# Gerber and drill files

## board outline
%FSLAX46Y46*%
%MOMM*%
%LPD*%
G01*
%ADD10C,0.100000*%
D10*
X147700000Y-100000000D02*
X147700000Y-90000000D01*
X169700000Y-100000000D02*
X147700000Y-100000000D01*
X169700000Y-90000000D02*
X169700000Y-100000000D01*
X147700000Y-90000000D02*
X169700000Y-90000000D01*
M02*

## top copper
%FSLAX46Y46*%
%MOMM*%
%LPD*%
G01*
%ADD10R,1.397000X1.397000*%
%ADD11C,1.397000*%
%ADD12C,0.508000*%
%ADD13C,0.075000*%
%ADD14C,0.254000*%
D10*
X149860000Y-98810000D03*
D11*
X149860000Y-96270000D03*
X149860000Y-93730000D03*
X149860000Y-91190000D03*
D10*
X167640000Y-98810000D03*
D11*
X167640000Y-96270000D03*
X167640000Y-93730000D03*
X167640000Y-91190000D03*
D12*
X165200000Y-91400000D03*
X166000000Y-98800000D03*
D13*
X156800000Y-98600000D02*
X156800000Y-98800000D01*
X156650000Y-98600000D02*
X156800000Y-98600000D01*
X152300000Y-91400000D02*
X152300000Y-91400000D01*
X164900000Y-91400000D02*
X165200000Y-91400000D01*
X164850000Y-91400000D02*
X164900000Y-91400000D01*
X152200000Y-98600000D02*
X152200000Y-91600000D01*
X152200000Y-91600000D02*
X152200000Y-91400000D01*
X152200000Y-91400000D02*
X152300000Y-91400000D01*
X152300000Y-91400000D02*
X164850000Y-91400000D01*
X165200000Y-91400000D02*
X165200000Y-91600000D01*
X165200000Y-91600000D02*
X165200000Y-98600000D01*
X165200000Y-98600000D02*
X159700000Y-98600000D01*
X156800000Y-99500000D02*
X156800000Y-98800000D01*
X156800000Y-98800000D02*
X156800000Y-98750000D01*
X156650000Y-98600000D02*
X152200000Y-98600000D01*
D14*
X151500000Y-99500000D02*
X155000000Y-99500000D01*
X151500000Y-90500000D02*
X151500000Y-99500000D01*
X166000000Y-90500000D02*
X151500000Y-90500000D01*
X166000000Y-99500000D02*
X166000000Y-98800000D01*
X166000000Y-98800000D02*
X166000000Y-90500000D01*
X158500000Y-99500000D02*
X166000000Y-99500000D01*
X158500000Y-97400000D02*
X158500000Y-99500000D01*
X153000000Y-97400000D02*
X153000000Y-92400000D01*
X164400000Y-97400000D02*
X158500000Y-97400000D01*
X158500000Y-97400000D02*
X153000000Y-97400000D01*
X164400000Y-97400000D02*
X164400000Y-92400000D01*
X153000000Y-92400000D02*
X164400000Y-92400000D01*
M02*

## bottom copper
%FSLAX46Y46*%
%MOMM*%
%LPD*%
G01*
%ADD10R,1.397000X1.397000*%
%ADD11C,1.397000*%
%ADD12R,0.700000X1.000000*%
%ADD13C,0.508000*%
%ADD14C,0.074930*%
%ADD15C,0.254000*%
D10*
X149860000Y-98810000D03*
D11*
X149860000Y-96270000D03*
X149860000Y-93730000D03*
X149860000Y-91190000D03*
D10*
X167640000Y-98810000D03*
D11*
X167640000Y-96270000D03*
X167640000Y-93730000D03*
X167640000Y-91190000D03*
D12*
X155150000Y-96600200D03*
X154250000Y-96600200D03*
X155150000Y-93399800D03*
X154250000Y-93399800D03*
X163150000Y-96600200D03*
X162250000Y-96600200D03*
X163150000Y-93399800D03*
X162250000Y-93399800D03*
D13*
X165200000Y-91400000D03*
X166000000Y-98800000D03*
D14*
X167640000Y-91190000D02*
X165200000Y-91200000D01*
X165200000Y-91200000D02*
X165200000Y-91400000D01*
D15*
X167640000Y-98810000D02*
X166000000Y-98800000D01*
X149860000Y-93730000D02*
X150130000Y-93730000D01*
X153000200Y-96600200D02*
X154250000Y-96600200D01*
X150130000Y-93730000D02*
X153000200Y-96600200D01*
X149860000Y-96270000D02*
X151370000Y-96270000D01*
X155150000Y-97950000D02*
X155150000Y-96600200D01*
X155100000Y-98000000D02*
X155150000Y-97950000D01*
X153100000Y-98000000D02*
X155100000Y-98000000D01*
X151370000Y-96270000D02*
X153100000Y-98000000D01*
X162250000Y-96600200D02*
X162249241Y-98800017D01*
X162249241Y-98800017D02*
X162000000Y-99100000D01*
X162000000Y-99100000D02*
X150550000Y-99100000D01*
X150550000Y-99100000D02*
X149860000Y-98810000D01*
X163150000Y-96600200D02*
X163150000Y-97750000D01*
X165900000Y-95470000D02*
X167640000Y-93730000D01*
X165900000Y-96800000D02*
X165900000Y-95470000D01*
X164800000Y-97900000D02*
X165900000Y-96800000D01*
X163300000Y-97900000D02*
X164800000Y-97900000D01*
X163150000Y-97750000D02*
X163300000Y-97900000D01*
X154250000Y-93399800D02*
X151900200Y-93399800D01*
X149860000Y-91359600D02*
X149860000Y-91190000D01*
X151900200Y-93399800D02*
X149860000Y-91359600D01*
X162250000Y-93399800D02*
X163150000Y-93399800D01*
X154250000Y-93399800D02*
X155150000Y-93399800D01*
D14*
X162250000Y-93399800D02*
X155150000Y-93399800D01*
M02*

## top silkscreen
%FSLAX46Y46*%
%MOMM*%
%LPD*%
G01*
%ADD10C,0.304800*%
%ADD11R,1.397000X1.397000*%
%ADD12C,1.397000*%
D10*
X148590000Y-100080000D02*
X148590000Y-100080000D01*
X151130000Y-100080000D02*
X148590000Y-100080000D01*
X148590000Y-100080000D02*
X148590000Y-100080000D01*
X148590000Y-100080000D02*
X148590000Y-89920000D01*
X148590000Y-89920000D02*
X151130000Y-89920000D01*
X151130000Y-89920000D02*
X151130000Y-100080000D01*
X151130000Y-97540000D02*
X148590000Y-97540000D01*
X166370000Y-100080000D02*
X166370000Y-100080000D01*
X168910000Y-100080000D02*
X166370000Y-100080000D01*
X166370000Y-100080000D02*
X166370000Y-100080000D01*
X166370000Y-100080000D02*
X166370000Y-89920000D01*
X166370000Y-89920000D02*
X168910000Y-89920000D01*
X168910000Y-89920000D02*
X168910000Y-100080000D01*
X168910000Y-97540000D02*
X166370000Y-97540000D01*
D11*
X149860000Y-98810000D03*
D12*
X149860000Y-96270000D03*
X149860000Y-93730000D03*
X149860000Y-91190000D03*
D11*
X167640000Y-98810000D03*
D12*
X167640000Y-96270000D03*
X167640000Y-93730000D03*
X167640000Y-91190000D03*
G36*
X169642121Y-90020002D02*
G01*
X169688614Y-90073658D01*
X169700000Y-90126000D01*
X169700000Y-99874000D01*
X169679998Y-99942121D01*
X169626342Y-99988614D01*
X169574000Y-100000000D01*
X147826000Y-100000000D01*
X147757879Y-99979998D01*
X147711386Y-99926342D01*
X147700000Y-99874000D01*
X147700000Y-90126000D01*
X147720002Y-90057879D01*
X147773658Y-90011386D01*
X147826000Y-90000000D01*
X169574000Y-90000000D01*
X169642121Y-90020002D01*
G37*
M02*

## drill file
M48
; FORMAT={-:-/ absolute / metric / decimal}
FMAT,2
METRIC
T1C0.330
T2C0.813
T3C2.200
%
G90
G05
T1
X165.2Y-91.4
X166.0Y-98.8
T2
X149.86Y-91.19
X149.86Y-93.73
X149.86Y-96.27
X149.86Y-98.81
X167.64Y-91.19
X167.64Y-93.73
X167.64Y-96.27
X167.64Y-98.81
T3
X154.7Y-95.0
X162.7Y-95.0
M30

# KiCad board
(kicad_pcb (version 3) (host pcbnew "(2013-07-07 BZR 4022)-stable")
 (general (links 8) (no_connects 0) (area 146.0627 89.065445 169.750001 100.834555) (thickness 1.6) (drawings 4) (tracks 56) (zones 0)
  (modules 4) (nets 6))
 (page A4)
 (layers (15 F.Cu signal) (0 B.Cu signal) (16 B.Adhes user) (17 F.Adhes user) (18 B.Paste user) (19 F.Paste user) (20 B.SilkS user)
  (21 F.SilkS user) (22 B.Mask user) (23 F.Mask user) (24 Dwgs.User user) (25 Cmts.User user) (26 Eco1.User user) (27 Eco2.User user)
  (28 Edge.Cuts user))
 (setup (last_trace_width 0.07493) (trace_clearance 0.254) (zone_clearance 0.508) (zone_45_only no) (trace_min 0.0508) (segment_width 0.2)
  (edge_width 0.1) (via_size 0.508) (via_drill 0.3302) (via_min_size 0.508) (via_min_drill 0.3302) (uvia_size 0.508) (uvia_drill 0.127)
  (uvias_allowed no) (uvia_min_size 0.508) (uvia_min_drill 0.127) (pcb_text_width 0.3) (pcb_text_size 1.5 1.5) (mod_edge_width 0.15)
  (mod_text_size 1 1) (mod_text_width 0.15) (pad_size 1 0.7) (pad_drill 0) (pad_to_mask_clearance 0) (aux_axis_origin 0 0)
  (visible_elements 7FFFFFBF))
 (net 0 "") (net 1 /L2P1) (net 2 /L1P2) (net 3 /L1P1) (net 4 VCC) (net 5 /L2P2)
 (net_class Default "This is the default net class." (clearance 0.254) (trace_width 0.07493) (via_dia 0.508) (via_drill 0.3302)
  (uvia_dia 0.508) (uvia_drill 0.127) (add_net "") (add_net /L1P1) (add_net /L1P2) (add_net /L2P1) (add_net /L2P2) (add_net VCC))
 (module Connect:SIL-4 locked (layer F.Cu) (at 149.86 95 90)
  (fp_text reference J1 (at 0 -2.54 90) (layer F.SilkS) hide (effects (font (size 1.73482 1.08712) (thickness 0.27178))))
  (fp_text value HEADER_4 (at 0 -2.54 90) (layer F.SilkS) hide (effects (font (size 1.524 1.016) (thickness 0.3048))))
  (fp_line (start -5.08 -1.27) (end -5.08 -1.27) (layer F.SilkS) (width 0.3048))
  (fp_line (start -5.08 1.27) (end -5.08 -1.27) (layer F.SilkS) (width 0.3048))
  (fp_line (start -5.08 -1.27) (end -5.08 -1.27) (layer F.SilkS) (width 0.3048))
  (fp_line (start -5.08 -1.27) (end 5.08 -1.27) (layer F.SilkS) (width 0.3048))
  (fp_line (start 5.08 -1.27) (end 5.08 1.27) (layer F.SilkS) (width 0.3048))
  (fp_line (start 5.08 1.27) (end -5.08 1.27) (layer F.SilkS) (width 0.3048))
  (fp_line (start -2.54 1.27) (end -2.54 -1.27) (layer F.SilkS) (width 0.3048))
  (pad 1 thru_hole rect (at -3.81 0 90) (size 1.397 1.397) (drill 0.8128) (layers *.Cu *.Mask F.SilkS) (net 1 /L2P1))
  (pad 2 thru_hole circle (at -1.27 0 90) (size 1.397 1.397) (drill 0.8128) (layers *.Cu *.Mask F.SilkS) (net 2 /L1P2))
  (pad 3 thru_hole circle (at 1.27 0 90) (size 1.397 1.397) (drill 0.8128) (layers *.Cu *.Mask F.SilkS) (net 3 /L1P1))
  (pad 4 thru_hole circle (at 3.81 0 90) (size 1.397 1.397) (drill 0.8128) (layers *.Cu *.Mask F.SilkS) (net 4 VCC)))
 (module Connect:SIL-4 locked (layer F.Cu) (at 167.64 95 90)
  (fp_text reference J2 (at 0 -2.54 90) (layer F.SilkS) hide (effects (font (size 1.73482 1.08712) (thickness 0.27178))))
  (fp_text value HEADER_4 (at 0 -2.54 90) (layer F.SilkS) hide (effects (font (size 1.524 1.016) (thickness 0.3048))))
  (fp_line (start -5.08 -1.27) (end -5.08 -1.27) (layer F.SilkS) (width 0.3048))
  (fp_line (start -5.08 1.27) (end -5.08 -1.27) (layer F.SilkS) (width 0.3048))
  (fp_line (start -5.08 -1.27) (end -5.08 -1.27) (layer F.SilkS) (width 0.3048))
  (fp_line (start -5.08 -1.27) (end 5.08 -1.27) (layer F.SilkS) (width 0.3048))
  (fp_line (start 5.08 -1.27) (end 5.08 1.27) (layer F.SilkS) (width 0.3048))
  (fp_line (start 5.08 1.27) (end -5.08 1.27) (layer F.SilkS) (width 0.3048))
  (fp_line (start -2.54 1.27) (end -2.54 -1.27) (layer F.SilkS) (width 0.3048))
  (pad 1 thru_hole rect (at -3.81 0 90) (size 1.397 1.397) (drill 0.8128) (layers *.Cu *.Mask F.SilkS))
  (pad 2 thru_hole circle (at -1.27 0 90) (size 1.397 1.397) (drill 0.8128) (layers *.Cu *.Mask F.SilkS))
  (pad 3 thru_hole circle (at 1.27 0 90) (size 1.397 1.397) (drill 0.8128) (layers *.Cu *.Mask F.SilkS) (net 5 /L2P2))
  (pad 4 thru_hole circle (at 3.81 0 90) (size 1.397 1.397) (drill 0.8128) (layers *.Cu *.Mask F.SilkS)))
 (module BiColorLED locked (layer B.Cu) (at 154.7 95 90)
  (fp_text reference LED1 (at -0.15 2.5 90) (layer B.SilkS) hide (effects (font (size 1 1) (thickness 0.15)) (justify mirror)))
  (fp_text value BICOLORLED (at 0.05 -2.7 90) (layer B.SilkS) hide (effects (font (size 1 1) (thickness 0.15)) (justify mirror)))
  (pad "" np_thru_hole circle (at 0 0 90) (size 2.2 2.2) (drill 2.2) (layers *.Cu *.Mask B.SilkS))
  (pad 2 smd rect (at -1.6002 0.45 90) (size 1 0.7) (layers B.Cu B.Paste B.Mask) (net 2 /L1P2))
  (pad 1 smd rect (at -1.6002 -0.45 90) (size 1 0.7) (layers B.Cu B.Paste B.Mask) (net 3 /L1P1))
  (pad 3 smd rect (at 1.6002 0.45 90) (size 1 0.7) (layers B.Cu B.Paste B.Mask) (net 4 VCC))
  (pad 4 smd rect (at 1.6002 -0.45 90) (size 1 0.7) (layers B.Cu B.Paste B.Mask) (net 4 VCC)))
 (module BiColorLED (layer B.Cu) (at 162.7 95 90)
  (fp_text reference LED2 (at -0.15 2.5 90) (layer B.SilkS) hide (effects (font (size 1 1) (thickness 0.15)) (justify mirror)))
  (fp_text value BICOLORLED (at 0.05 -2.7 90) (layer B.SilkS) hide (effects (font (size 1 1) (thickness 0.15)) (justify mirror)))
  (pad "" np_thru_hole circle (at 0 0 90) (size 2.2 2.2) (drill 2.2) (layers *.Cu *.Mask B.SilkS))
  (pad 2 smd rect (at -1.6002 0.45 90) (size 1 0.7) (layers B.Cu B.Paste B.Mask) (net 5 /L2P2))
  (pad 1 smd rect (at -1.6002 -0.45 90) (size 1 0.7) (layers B.Cu B.Paste B.Mask) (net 1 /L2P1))
  (pad 3 smd rect (at 1.6002 0.45 90) (size 1 0.7) (layers B.Cu B.Paste B.Mask) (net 4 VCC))
  (pad 4 smd rect (at 1.6002 -0.45 90) (size 1 0.7) (layers B.Cu B.Paste B.Mask) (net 4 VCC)))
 (gr_line (start 147.7 100) (end 147.7 90) (angle 90) (layer Edge.Cuts) (width 0.1))
 (gr_line (start 169.7 100) (end 147.7 100) (angle 90) (layer Edge.Cuts) (width 0.1))
 (gr_line (start 169.7 90) (end 169.7 100) (angle 90) (layer Edge.Cuts) (width 0.1))
 (gr_line (start 147.7 90) (end 169.7 90) (angle 90) (layer Edge.Cuts) (width 0.1))
 (segment (start 167.64 91.19) (end 165.2 91.2) (width 0.07493) (layer B.Cu) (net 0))
 (segment (start 165.2 91.2) (end 165.2 91.4) (width 0.07493) (layer B.Cu) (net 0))
 (via (at 165.2 91.4) (size 0.508) (layers F.Cu B.Cu) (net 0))
 (segment (start 167.64 98.81) (end 166 98.8) (width 0.254) (layer B.Cu) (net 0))
 (via (at 166 98.8) (size 0.508) (layers F.Cu B.Cu) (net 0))
 (segment (start 156.8 98.6) (end 156.8 98.8) (width 0.075) (layer F.Cu) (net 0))
 (segment (start 156.65 98.6) (end 156.8 98.6) (width 0.075) (layer F.Cu) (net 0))
 (segment (start 152.3 91.4) (end 152.3 91.4) (width 0.075) (layer F.Cu) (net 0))
 (segment (start 164.9 91.4) (end 165.2 91.4) (width 0.075) (layer F.Cu) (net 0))
 (segment (start 164.85 91.4) (end 164.9 91.4) (width 0.075) (layer F.Cu) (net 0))
 (segment (start 152.2 98.6) (end 152.2 91.6) (width 0.075) (layer F.Cu) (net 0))
 (segment (start 152.2 91.6) (end 152.2 91.4) (width 0.075) (layer F.Cu) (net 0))
 (segment (start 152.2 91.4) (end 152.3 91.4) (width 0.075) (layer F.Cu) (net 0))
 (segment (start 152.3 91.4) (end 164.85 91.4) (width 0.075) (layer F.Cu) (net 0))
 (segment (start 165.2 91.4) (end 165.2 91.6) (width 0.075) (layer F.Cu) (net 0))
 (segment (start 165.2 91.6) (end 165.2 98.6) (width 0.075) (layer F.Cu) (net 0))
 (segment (start 165.2 98.6) (end 159.7 98.6) (width 0.075) (layer F.Cu) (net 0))
 (segment (start 156.8 99.5) (end 156.8 98.8) (width 0.075) (layer F.Cu) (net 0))
 (segment (start 156.8 98.8) (end 156.8 98.75) (width 0.075) (layer F.Cu) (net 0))
 (segment (start 156.65 98.6) (end 152.2 98.6) (width 0.075) (layer F.Cu) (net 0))
 (segment (start 151.5 99.5) (end 155 99.5) (width 0.254) (layer F.Cu) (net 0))
 (segment (start 151.5 90.5) (end 151.5 99.5) (width 0.254) (layer F.Cu) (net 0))
 (segment (start 166 90.5) (end 151.5 90.5) (width 0.254) (layer F.Cu) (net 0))
 (segment (start 166 99.5) (end 166 98.8) (width 0.254) (layer F.Cu) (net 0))
 (segment (start 166 98.8) (end 166 90.5) (width 0.254) (layer F.Cu) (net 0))
 (segment (start 158.5 99.5) (end 166 99.5) (width 0.254) (layer F.Cu) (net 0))
 (segment (start 158.5 97.4) (end 158.5 99.5) (width 0.254) (layer F.Cu) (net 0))
 (segment (start 153 97.4) (end 153 92.4) (width 0.254) (layer F.Cu) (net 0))
 (segment (start 164.4 97.4) (end 158.5 97.4) (width 0.254) (layer F.Cu) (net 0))
 (segment (start 158.5 97.4) (end 153 97.4) (width 0.254) (layer F.Cu) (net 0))
 (segment (start 164.4 97.4) (end 164.4 92.4) (width 0.254) (layer F.Cu) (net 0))
 (segment (start 153 92.4) (end 164.4 92.4) (width 0.254) (layer F.Cu) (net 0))
 (segment (start 149.86 93.73) (end 150.13 93.73) (width 0.254) (layer B.Cu) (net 3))
 (segment (start 153.0002 96.6002) (end 154.25 96.6002) (width 0.254) (layer B.Cu) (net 3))
 (segment (start 150.13 93.73) (end 153.0002 96.6002) (width 0.254) (layer B.Cu) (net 3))
 (segment (start 149.86 96.27) (end 151.37 96.27) (width 0.254) (layer B.Cu) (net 2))
 (segment (start 155.15 97.95) (end 155.15 96.6002) (width 0.254) (layer B.Cu) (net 2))
 (segment (start 155.1 98) (end 155.15 97.95) (width 0.254) (layer B.Cu) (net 2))
 (segment (start 153.1 98) (end 155.1 98) (width 0.254) (layer B.Cu) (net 2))
 (segment (start 151.37 96.27) (end 153.1 98) (width 0.254) (layer B.Cu) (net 2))
 (segment (start 162.25 96.6002) (end 162.249241 98.800017) (width 0.254) (layer B.Cu) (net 1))
 (segment (start 162.249241 98.800017) (end 162 99.1) (width 0.254) (layer B.Cu) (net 1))
 (segment (start 162 99.1) (end 150.55 99.1) (width 0.254) (layer B.Cu) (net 1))
 (segment (start 150.55 99.1) (end 149.86 98.81) (width 0.254) (layer B.Cu) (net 1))
 (segment (start 163.15 96.6002) (end 163.15 97.75) (width 0.254) (layer B.Cu) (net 5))
 (segment (start 165.9 95.47) (end 167.64 93.73) (width 0.254) (layer B.Cu) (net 5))
 (segment (start 165.9 96.8) (end 165.9 95.47) (width 0.254) (layer B.Cu) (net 5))
 (segment (start 164.8 97.9) (end 165.9 96.8) (width 0.254) (layer B.Cu) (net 5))
 (segment (start 163.3 97.9) (end 164.8 97.9) (width 0.254) (layer B.Cu) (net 5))
 (segment (start 163.15 97.75) (end 163.3 97.9) (width 0.254) (layer B.Cu) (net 5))
 (segment (start 154.25 93.3998) (end 151.9002 93.3998) (width 0.254) (layer B.Cu) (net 4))
 (segment (start 149.86 91.3596) (end 149.86 91.19) (width 0.254) (layer B.Cu) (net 4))
 (segment (start 151.9002 93.3998) (end 149.86 91.3596) (width 0.254) (layer B.Cu) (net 4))
 (segment (start 162.25 93.3998) (end 163.15 93.3998) (width 0.254) (layer B.Cu) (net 4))
 (segment (start 154.25 93.3998) (end 155.15 93.3998) (width 0.254) (layer B.Cu) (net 4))
 (segment (start 162.25 93.3998) (end 155.15 93.3998) (width 0.07493) (layer B.Cu) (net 4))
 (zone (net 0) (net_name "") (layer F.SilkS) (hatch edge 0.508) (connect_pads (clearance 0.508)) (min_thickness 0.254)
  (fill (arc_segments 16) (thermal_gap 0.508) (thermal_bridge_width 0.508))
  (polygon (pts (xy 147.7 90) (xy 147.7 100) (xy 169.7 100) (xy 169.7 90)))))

